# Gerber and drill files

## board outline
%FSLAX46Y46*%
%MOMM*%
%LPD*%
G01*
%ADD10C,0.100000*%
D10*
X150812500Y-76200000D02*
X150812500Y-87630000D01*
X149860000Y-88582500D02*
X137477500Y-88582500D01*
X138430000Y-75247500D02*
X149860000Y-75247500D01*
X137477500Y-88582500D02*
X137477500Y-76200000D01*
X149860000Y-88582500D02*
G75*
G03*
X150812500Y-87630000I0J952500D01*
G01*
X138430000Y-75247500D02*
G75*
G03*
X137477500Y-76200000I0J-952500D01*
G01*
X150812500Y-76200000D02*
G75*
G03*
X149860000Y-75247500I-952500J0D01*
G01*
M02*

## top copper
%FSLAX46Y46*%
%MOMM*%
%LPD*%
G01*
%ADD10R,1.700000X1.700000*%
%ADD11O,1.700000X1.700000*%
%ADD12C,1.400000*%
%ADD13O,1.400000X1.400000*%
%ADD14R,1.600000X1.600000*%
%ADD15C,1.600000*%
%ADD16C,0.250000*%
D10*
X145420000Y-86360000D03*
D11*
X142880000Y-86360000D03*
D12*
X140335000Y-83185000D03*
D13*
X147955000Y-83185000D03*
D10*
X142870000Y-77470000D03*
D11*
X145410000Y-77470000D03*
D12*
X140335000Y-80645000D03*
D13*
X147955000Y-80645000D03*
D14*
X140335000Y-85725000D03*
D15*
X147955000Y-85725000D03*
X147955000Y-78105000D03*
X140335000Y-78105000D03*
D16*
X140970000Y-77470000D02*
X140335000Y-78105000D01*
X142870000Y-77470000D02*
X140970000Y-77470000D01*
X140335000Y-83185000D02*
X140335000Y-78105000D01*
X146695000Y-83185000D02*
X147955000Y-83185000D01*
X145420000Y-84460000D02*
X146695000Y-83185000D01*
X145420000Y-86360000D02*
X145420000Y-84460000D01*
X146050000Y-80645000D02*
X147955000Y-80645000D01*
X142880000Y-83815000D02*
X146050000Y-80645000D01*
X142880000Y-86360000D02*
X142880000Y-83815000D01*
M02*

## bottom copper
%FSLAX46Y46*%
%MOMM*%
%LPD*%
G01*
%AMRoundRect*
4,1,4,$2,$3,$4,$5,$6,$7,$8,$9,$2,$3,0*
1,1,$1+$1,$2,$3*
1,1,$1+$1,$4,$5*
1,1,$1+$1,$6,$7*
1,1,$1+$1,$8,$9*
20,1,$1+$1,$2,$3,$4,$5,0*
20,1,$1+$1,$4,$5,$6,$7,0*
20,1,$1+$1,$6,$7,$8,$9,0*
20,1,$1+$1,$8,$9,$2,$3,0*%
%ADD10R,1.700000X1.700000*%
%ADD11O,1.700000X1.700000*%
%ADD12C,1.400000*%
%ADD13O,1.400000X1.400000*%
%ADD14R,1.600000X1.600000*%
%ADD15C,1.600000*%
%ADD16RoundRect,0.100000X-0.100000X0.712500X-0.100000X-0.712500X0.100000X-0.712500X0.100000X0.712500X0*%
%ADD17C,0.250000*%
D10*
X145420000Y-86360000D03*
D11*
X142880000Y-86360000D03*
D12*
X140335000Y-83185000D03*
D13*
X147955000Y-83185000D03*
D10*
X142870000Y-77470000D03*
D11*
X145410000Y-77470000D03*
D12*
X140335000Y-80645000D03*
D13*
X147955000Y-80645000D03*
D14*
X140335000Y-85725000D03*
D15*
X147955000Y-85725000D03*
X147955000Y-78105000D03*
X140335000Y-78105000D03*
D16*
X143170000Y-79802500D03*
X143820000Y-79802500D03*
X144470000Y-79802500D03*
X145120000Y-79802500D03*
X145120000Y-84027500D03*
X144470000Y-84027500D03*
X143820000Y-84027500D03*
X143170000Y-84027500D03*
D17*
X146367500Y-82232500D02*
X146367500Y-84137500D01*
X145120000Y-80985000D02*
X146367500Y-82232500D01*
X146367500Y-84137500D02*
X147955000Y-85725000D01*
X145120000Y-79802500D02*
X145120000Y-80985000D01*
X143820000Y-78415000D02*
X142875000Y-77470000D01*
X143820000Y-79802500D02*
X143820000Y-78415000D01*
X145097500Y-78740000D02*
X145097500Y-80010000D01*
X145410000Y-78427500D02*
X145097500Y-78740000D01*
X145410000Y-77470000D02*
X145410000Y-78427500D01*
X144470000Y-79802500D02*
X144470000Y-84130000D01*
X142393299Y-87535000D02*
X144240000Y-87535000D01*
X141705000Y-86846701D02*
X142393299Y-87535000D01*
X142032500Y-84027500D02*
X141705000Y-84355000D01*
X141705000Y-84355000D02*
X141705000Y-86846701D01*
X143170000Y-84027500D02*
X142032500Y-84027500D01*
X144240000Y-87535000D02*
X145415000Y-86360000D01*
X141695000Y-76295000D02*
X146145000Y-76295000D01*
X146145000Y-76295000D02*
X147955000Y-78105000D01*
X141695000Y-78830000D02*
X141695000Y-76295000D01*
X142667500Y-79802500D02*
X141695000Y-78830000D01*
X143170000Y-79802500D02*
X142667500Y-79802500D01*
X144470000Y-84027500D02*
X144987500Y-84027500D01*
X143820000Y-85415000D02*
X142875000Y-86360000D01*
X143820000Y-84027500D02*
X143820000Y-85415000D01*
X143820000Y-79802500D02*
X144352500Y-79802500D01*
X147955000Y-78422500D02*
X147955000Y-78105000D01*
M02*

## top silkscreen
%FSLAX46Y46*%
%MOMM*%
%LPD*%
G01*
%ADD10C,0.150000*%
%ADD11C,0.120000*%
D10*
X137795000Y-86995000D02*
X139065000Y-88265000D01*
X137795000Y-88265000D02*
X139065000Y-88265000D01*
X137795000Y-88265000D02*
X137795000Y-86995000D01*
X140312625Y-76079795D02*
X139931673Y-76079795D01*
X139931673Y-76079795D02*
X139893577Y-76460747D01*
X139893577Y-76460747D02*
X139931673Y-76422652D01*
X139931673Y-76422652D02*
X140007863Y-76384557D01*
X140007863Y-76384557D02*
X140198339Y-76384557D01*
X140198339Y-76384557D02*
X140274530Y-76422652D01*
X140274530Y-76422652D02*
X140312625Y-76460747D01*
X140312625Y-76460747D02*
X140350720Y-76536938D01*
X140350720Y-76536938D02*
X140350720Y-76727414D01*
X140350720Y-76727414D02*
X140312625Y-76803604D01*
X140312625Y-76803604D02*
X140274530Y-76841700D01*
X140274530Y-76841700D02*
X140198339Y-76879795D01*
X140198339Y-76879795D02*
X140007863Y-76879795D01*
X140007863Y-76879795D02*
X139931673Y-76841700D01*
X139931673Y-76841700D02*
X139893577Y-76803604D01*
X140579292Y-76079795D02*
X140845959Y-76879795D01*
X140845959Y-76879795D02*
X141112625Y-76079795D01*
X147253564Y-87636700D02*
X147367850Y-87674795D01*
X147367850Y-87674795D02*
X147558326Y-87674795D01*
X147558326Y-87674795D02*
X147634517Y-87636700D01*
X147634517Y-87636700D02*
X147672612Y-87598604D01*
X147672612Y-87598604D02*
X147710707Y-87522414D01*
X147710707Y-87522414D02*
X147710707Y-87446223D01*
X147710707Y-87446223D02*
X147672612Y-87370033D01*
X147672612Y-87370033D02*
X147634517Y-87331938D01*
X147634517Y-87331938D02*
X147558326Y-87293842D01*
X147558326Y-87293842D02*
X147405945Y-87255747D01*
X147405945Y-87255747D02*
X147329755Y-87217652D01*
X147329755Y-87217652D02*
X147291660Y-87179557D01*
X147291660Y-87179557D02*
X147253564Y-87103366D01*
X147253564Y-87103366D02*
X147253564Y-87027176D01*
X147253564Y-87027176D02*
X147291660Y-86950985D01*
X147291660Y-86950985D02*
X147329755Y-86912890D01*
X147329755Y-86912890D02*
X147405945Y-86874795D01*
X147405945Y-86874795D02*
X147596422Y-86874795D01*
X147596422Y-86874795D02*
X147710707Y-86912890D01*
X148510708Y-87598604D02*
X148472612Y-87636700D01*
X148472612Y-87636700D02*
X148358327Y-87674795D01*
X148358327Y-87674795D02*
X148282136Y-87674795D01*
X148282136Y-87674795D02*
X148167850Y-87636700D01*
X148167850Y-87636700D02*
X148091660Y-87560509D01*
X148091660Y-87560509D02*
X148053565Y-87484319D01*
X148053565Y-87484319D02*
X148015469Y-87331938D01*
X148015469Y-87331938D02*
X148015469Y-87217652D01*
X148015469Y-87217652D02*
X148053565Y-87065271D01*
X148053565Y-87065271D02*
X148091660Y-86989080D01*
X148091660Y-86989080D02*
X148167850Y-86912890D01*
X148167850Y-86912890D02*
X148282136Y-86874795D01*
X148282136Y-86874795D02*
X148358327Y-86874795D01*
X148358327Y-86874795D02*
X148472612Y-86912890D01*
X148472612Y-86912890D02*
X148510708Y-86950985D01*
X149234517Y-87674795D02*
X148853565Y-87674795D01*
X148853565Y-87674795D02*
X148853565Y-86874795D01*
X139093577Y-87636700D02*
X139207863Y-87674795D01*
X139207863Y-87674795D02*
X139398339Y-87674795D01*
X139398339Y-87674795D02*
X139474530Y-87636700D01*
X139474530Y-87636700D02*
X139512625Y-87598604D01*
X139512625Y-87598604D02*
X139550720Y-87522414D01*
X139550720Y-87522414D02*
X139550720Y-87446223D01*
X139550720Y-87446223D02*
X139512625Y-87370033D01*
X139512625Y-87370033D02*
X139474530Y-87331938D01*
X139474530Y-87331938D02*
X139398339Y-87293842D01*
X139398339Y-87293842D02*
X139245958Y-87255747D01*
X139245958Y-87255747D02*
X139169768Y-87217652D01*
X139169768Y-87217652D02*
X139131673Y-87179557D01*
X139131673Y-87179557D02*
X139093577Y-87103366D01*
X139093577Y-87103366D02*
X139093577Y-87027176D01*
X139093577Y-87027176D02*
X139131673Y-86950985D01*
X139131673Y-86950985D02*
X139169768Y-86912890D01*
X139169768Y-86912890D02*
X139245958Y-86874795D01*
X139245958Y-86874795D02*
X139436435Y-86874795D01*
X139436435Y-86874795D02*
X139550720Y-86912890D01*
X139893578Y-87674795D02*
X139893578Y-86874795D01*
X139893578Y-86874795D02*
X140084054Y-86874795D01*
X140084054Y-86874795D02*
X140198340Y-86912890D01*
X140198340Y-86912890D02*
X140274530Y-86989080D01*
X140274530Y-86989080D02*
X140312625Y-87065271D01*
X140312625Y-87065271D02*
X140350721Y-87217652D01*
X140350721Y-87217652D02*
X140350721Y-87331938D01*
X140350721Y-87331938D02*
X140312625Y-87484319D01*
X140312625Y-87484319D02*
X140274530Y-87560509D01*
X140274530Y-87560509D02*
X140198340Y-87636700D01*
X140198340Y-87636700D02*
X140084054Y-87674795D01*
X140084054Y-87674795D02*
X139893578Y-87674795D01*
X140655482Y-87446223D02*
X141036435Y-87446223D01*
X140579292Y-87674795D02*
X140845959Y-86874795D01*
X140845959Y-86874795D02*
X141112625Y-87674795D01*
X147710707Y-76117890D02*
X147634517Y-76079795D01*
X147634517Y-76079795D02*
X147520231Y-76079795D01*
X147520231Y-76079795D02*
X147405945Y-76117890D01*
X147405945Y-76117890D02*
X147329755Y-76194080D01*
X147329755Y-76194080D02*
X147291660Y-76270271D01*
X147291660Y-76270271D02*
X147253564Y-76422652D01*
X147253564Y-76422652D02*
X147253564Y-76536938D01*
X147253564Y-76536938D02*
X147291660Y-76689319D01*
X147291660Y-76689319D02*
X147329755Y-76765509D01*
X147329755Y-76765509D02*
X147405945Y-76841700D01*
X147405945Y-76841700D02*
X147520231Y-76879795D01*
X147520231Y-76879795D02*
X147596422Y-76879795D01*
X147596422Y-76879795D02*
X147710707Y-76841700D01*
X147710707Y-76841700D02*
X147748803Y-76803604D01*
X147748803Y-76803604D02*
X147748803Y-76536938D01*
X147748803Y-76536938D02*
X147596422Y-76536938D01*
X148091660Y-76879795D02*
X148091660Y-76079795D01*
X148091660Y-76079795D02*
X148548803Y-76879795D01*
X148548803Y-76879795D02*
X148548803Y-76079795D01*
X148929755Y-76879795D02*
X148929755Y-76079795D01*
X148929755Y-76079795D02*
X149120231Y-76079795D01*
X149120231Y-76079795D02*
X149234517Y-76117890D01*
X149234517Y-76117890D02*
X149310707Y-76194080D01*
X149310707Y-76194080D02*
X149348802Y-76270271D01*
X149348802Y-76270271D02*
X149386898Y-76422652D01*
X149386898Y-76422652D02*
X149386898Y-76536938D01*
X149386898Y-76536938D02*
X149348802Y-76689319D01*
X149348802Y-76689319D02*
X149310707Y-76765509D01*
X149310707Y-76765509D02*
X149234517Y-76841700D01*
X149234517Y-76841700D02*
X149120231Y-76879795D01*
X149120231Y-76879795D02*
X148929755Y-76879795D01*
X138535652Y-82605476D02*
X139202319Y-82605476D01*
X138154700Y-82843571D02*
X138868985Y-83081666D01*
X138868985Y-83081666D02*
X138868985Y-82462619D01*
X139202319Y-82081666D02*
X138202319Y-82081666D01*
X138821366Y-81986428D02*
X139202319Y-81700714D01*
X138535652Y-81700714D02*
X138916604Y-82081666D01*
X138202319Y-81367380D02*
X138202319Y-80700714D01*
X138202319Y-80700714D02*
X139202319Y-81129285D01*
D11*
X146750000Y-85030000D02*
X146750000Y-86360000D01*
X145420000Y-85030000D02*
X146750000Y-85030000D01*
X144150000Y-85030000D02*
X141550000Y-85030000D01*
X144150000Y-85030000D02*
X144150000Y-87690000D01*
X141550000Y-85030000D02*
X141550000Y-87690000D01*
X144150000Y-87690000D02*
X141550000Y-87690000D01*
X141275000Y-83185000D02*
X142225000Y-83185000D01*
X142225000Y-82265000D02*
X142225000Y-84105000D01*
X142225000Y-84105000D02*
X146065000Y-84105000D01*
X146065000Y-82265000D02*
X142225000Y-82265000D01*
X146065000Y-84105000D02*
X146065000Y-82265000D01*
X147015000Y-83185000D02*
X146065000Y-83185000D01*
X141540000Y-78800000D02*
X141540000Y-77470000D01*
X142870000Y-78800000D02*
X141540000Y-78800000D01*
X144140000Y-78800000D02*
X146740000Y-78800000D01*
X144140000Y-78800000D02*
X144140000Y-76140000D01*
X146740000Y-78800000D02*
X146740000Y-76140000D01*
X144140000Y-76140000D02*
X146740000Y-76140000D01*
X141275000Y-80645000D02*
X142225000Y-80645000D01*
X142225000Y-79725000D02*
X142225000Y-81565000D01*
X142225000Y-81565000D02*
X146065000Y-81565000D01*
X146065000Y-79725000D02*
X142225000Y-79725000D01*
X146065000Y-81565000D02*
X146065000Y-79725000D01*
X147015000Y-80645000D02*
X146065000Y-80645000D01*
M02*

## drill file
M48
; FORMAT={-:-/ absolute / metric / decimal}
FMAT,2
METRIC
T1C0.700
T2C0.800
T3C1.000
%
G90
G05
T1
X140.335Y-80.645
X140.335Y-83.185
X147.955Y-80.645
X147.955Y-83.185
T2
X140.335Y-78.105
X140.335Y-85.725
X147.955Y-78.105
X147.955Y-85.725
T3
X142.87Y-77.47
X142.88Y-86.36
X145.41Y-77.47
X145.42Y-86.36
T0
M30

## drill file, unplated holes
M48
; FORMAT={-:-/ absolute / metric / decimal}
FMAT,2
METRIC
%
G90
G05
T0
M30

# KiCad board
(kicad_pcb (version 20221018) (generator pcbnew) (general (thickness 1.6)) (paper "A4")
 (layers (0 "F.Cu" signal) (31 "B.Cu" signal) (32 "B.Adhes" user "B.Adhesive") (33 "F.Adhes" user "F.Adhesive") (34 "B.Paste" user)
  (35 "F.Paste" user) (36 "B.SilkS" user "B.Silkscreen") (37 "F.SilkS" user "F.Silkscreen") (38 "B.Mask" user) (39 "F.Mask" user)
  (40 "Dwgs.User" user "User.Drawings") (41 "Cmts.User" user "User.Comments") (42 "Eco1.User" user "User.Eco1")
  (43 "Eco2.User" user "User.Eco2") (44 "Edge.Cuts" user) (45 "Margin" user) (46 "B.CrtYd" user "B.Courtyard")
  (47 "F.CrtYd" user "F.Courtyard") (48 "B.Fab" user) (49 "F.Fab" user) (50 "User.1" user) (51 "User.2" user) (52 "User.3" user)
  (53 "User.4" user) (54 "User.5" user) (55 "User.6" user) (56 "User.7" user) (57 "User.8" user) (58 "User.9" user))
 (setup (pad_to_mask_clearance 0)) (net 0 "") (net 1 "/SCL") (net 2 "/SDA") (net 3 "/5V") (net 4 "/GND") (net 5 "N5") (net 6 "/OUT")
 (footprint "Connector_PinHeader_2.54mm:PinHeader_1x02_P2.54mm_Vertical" (layer "F.Cu") (at 145.42 86.36 -90)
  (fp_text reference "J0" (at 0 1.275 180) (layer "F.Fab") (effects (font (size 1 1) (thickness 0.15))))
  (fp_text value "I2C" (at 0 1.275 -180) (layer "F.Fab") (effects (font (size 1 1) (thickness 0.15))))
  (fp_line (start -1.33 -1.33) (end 0 -1.33) (stroke (width 0.12) (type solid)) (layer "F.SilkS"))
  (fp_line (start -1.33 0) (end -1.33 -1.33) (stroke (width 0.12) (type solid)) (layer "F.SilkS"))
  (fp_line (start -1.33 1.27) (end -1.33 3.87) (stroke (width 0.12) (type solid)) (layer "F.SilkS"))
  (fp_line (start -1.33 1.27) (end 1.33 1.27) (stroke (width 0.12) (type solid)) (layer "F.SilkS"))
  (fp_line (start -1.33 3.87) (end 1.33 3.87) (stroke (width 0.12) (type solid)) (layer "F.SilkS"))
  (fp_line (start 1.33 1.27) (end 1.33 3.87) (stroke (width 0.12) (type solid)) (layer "F.SilkS"))
  (pad "1" thru_hole rect (at 0 0 270) (size 1.7 1.7) (drill 1) (layers "*.Cu" "*.Mask") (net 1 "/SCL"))
  (pad "2" thru_hole oval (at 0 2.54 270) (size 1.7 1.7) (drill 1) (layers "*.Cu" "*.Mask") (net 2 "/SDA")))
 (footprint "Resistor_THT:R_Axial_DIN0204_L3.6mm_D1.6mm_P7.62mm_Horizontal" (layer "F.Cu") (at 140.335 83.185)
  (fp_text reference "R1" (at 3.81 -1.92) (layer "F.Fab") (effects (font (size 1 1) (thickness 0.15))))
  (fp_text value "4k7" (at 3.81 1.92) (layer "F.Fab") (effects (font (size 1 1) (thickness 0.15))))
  (fp_line (start 0.94 0) (end 1.89 0) (stroke (width 0.12) (type solid)) (layer "F.SilkS"))
  (fp_line (start 1.89 -0.92) (end 1.89 0.92) (stroke (width 0.12) (type solid)) (layer "F.SilkS"))
  (fp_line (start 1.89 0.92) (end 5.73 0.92) (stroke (width 0.12) (type solid)) (layer "F.SilkS"))
  (fp_line (start 5.73 -0.92) (end 1.89 -0.92) (stroke (width 0.12) (type solid)) (layer "F.SilkS"))
  (fp_line (start 5.73 0.92) (end 5.73 -0.92) (stroke (width 0.12) (type solid)) (layer "F.SilkS"))
  (fp_line (start 6.68 0) (end 5.73 0) (stroke (width 0.12) (type solid)) (layer "F.SilkS"))
  (pad "1" thru_hole circle (at 0 0) (size 1.4 1.4) (drill 0.7) (layers "*.Cu" "*.Mask") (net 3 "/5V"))
  (pad "2" thru_hole oval (at 7.62 0) (size 1.4 1.4) (drill 0.7) (layers "*.Cu" "*.Mask") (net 1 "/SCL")))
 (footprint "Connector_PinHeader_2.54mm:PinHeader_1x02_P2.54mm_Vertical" (layer "F.Cu") (at 142.87 77.47 90)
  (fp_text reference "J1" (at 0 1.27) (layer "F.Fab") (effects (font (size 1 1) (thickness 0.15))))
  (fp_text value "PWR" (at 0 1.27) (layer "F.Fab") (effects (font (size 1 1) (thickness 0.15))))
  (fp_line (start -1.33 -1.33) (end 0 -1.33) (stroke (width 0.12) (type solid)) (layer "F.SilkS"))
  (fp_line (start -1.33 0) (end -1.33 -1.33) (stroke (width 0.12) (type solid)) (layer "F.SilkS"))
  (fp_line (start -1.33 1.27) (end -1.33 3.87) (stroke (width 0.12) (type solid)) (layer "F.SilkS"))
  (fp_line (start -1.33 1.27) (end 1.33 1.27) (stroke (width 0.12) (type solid)) (layer "F.SilkS"))
  (fp_line (start -1.33 3.87) (end 1.33 3.87) (stroke (width 0.12) (type solid)) (layer "F.SilkS"))
  (fp_line (start 1.33 1.27) (end 1.33 3.87) (stroke (width 0.12) (type solid)) (layer "F.SilkS"))
  (pad "1" thru_hole rect (at 0 0 90) (size 1.7 1.7) (drill 1) (layers "*.Cu" "*.Mask") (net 3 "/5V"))
  (pad "2" thru_hole oval (at 0 2.54 90) (size 1.7 1.7) (drill 1) (layers "*.Cu" "*.Mask") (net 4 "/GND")))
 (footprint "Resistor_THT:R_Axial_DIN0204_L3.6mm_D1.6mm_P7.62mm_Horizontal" (layer "F.Cu") (at 140.335 80.645)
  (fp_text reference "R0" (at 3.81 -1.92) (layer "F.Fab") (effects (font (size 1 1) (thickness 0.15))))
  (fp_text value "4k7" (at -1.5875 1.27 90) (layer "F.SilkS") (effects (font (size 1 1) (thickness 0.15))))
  (fp_line (start 0.94 0) (end 1.89 0) (stroke (width 0.12) (type solid)) (layer "F.SilkS"))
  (fp_line (start 1.89 -0.92) (end 1.89 0.92) (stroke (width 0.12) (type solid)) (layer "F.SilkS"))
  (fp_line (start 1.89 0.92) (end 5.73 0.92) (stroke (width 0.12) (type solid)) (layer "F.SilkS"))
  (fp_line (start 5.73 -0.92) (end 1.89 -0.92) (stroke (width 0.12) (type solid)) (layer "F.SilkS"))
  (fp_line (start 5.73 0.92) (end 5.73 -0.92) (stroke (width 0.12) (type solid)) (layer "F.SilkS"))
  (fp_line (start 6.68 0) (end 5.73 0) (stroke (width 0.12) (type solid)) (layer "F.SilkS"))
  (pad "1" thru_hole circle (at 0 0) (size 1.4 1.4) (drill 0.7) (layers "*.Cu" "*.Mask") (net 3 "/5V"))
  (pad "2" thru_hole oval (at 7.62 0) (size 1.4 1.4) (drill 0.7) (layers "*.Cu" "*.Mask") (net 2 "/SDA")))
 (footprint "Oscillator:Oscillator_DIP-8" (layer "F.Cu") (at 140.335 85.725)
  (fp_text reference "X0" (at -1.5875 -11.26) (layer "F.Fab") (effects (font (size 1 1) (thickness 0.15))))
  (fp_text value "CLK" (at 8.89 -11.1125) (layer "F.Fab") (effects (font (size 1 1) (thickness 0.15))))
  (pad "1" thru_hole rect (at 0 0) (size 1.6 1.6) (drill 0.8) (layers "*.Cu" "*.Mask") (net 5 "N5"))
  (pad "4" thru_hole circle (at 7.62 0) (size 1.6 1.6) (drill 0.8) (layers "*.Cu" "*.Mask") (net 4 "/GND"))
  (pad "5" thru_hole circle (at 7.62 -7.62) (size 1.6 1.6) (drill 0.8) (layers "*.Cu" "*.Mask") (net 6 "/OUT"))
  (pad "8" thru_hole circle (at 0 -7.62) (size 1.6 1.6) (drill 0.8) (layers "*.Cu" "*.Mask") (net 3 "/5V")))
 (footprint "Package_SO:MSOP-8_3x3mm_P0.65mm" (layer "B.Cu") (at 144.145 81.915 -90)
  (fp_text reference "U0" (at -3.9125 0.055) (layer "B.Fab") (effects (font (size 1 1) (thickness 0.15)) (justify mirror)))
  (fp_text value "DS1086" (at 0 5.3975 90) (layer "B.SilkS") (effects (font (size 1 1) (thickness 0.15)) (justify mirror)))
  (pad "1" smd roundrect (at -2.1125 0.975 270) (size 1.625 0.4) (layers "B.Cu" "B.Paste" "B.Mask") (roundrect_rratio 0.25) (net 6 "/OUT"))
  (pad "2" smd roundrect (at -2.1125 0.325 270) (size 1.625 0.4) (layers "B.Cu" "B.Paste" "B.Mask") (roundrect_rratio 0.25) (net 3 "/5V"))
  (pad "3" smd roundrect (at -2.1125 -0.325 270) (size 1.625 0.4) (layers "B.Cu" "B.Paste" "B.Mask") (roundrect_rratio 0.25) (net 3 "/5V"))
  (pad "4" smd roundrect (at -2.1125 -0.975 270) (size 1.625 0.4) (layers "B.Cu" "B.Paste" "B.Mask") (roundrect_rratio 0.25) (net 4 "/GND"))
  (pad "5" smd roundrect (at 2.1125 -0.975 270) (size 1.625 0.4) (layers "B.Cu" "B.Paste" "B.Mask") (roundrect_rratio 0.25) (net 3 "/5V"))
  (pad "6" smd roundrect (at 2.1125 -0.325 270) (size 1.625 0.4) (layers "B.Cu" "B.Paste" "B.Mask") (roundrect_rratio 0.25) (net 3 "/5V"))
  (pad "7" smd roundrect (at 2.1125 0.325 270) (size 1.625 0.4) (layers "B.Cu" "B.Paste" "B.Mask") (roundrect_rratio 0.25) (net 2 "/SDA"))
  (pad "8" smd roundrect (at 2.1125 0.975 270) (size 1.625 0.4) (layers "B.Cu" "B.Paste" "B.Mask") (roundrect_rratio 0.25) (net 1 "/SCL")))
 (gr_line (start 137.795 88.265) (end 139.065 88.265) (stroke (width 0.15) (type default)) (layer "F.SilkS"))
 (gr_line (start 137.795 86.995) (end 139.065 88.265) (stroke (width 0.15) (type default)) (layer "F.SilkS"))
 (gr_line (start 137.795 88.265) (end 137.795 86.995) (stroke (width 0.15) (type default)) (layer "F.SilkS"))
 (gr_line (start 150.8125 76.2) (end 150.8125 87.63) (stroke (width 0.1) (type default)) (layer "Edge.Cuts"))
 (gr_line (start 149.86 88.5825) (end 137.4775 88.5825) (stroke (width 0.1) (type default)) (layer "Edge.Cuts"))
 (gr_line (start 138.43 75.2475) (end 149.86 75.2475) (stroke (width 0.1) (type default)) (layer "Edge.Cuts"))
 (gr_line (start 137.4775 88.5825) (end 137.4775 76.2) (stroke (width 0.1) (type default)) (layer "Edge.Cuts"))
 (gr_arc (start 150.8125 87.63) (mid 150.533519 88.303519) (end 149.86 88.5825) (stroke (width 0.1) (type default)) (layer "Edge.Cuts"))
 (gr_arc (start 137.4775 76.2) (mid 137.756481 75.526481) (end 138.43 75.2475) (stroke (width 0.1) (type default)) (layer "Edge.Cuts"))
 (gr_arc (start 149.86 75.2475) (mid 150.533519 75.526481) (end 150.8125 76.2) (stroke (width 0.1) (type default)) (layer "Edge.Cuts"))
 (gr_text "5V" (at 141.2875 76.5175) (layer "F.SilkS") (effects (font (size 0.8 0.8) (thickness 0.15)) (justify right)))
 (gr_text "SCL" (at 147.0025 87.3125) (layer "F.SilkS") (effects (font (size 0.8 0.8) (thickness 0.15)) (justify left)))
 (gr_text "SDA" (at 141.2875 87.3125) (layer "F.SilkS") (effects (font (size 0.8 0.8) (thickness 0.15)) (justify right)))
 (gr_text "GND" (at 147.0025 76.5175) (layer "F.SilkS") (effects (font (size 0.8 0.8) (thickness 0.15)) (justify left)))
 (segment (start 140.335 83.185) (end 140.335 78.105) (width 0.25) (layer "F.Cu") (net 3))
 (segment (start 140.97 77.47) (end 140.335 78.105) (width 0.25) (layer "F.Cu") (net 3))
 (segment (start 142.87 77.47) (end 140.97 77.47) (width 0.25) (layer "F.Cu") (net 3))
 (segment (start 143.82 79.8025) (end 143.82 78.415) (width 0.25) (layer "B.Cu") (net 3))
 (segment (start 143.82 79.8025) (end 144.3525 79.8025) (width 0.25) (layer "B.Cu") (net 3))
 (segment (start 144.47 84.0275) (end 144.9875 84.0275) (width 0.25) (layer "B.Cu") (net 3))
 (segment (start 143.82 78.415) (end 142.875 77.47) (width 0.25) (layer "B.Cu") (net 3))
 (segment (start 144.47 79.8025) (end 144.47 84.13) (width 0.25) (layer "B.Cu") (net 3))
 (segment (start 145.42 86.36) (end 145.42 84.46) (width 0.25) (layer "F.Cu") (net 1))
 (segment (start 146.695 83.185) (end 147.955 83.185) (width 0.25) (layer "F.Cu") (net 1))
 (segment (start 145.42 84.46) (end 146.695 83.185) (width 0.25) (layer "F.Cu") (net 1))
 (segment (start 143.17 84.0275) (end 142.0325 84.0275) (width 0.25) (layer "B.Cu") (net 1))
 (segment (start 142.393299 87.535) (end 144.24 87.535) (width 0.25) (layer "B.Cu") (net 1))
 (segment (start 142.0325 84.0275) (end 141.705 84.355) (width 0.25) (layer "B.Cu") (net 1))
 (segment (start 141.705 84.355) (end 141.705 86.846701) (width 0.25) (layer "B.Cu") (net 1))
 (segment (start 141.705 86.846701) (end 142.393299 87.535) (width 0.25) (layer "B.Cu") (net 1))
 (segment (start 144.24 87.535) (end 145.415 86.36) (width 0.25) (layer "B.Cu") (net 1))
 (segment (start 142.88 83.815) (end 146.05 80.645) (width 0.25) (layer "F.Cu") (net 2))
 (segment (start 146.05 80.645) (end 147.955 80.645) (width 0.25) (layer "F.Cu") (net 2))
 (segment (start 142.88 86.36) (end 142.88 83.815) (width 0.25) (layer "F.Cu") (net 2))
 (segment (start 143.82 85.415) (end 142.875 86.36) (width 0.25) (layer "B.Cu") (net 2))
 (segment (start 143.82 84.0275) (end 143.82 85.415) (width 0.25) (layer "B.Cu") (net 2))
 (segment (start 145.41 78.4275) (end 145.0975 78.74) (width 0.25) (layer "B.Cu") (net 4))
 (segment (start 145.12 79.8025) (end 145.12 80.985) (width 0.25) (layer "B.Cu") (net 4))
 (segment (start 146.3675 84.1375) (end 147.955 85.725) (width 0.25) (layer "B.Cu") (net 4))
 (segment (start 145.41 77.47) (end 145.41 78.4275) (width 0.25) (layer "B.Cu") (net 4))
 (segment (start 145.0975 78.74) (end 145.0975 80.01) (width 0.25) (layer "B.Cu") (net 4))
 (segment (start 146.3675 82.2325) (end 146.3675 84.1375) (width 0.25) (layer "B.Cu") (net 4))
 (segment (start 145.12 80.985) (end 146.3675 82.2325) (width 0.25) (layer "B.Cu") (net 4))
 (segment (start 146.145 76.295) (end 147.955 78.105) (width 0.25) (layer "B.Cu") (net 6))
 (segment (start 147.955 78.4225) (end 147.955 78.105) (width 0.25) (layer "B.Cu") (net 6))
 (segment (start 142.6675 79.8025) (end 141.695 78.83) (width 0.25) (layer "B.Cu") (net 6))
 (segment (start 141.695 76.295) (end 146.145 76.295) (width 0.25) (layer "B.Cu") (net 6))
 (segment (start 143.17 79.8025) (end 142.6675 79.8025) (width 0.25) (layer "B.Cu") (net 6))
 (segment (start 141.695 78.83) (end 141.695 76.295) (width 0.25) (layer "B.Cu") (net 6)))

